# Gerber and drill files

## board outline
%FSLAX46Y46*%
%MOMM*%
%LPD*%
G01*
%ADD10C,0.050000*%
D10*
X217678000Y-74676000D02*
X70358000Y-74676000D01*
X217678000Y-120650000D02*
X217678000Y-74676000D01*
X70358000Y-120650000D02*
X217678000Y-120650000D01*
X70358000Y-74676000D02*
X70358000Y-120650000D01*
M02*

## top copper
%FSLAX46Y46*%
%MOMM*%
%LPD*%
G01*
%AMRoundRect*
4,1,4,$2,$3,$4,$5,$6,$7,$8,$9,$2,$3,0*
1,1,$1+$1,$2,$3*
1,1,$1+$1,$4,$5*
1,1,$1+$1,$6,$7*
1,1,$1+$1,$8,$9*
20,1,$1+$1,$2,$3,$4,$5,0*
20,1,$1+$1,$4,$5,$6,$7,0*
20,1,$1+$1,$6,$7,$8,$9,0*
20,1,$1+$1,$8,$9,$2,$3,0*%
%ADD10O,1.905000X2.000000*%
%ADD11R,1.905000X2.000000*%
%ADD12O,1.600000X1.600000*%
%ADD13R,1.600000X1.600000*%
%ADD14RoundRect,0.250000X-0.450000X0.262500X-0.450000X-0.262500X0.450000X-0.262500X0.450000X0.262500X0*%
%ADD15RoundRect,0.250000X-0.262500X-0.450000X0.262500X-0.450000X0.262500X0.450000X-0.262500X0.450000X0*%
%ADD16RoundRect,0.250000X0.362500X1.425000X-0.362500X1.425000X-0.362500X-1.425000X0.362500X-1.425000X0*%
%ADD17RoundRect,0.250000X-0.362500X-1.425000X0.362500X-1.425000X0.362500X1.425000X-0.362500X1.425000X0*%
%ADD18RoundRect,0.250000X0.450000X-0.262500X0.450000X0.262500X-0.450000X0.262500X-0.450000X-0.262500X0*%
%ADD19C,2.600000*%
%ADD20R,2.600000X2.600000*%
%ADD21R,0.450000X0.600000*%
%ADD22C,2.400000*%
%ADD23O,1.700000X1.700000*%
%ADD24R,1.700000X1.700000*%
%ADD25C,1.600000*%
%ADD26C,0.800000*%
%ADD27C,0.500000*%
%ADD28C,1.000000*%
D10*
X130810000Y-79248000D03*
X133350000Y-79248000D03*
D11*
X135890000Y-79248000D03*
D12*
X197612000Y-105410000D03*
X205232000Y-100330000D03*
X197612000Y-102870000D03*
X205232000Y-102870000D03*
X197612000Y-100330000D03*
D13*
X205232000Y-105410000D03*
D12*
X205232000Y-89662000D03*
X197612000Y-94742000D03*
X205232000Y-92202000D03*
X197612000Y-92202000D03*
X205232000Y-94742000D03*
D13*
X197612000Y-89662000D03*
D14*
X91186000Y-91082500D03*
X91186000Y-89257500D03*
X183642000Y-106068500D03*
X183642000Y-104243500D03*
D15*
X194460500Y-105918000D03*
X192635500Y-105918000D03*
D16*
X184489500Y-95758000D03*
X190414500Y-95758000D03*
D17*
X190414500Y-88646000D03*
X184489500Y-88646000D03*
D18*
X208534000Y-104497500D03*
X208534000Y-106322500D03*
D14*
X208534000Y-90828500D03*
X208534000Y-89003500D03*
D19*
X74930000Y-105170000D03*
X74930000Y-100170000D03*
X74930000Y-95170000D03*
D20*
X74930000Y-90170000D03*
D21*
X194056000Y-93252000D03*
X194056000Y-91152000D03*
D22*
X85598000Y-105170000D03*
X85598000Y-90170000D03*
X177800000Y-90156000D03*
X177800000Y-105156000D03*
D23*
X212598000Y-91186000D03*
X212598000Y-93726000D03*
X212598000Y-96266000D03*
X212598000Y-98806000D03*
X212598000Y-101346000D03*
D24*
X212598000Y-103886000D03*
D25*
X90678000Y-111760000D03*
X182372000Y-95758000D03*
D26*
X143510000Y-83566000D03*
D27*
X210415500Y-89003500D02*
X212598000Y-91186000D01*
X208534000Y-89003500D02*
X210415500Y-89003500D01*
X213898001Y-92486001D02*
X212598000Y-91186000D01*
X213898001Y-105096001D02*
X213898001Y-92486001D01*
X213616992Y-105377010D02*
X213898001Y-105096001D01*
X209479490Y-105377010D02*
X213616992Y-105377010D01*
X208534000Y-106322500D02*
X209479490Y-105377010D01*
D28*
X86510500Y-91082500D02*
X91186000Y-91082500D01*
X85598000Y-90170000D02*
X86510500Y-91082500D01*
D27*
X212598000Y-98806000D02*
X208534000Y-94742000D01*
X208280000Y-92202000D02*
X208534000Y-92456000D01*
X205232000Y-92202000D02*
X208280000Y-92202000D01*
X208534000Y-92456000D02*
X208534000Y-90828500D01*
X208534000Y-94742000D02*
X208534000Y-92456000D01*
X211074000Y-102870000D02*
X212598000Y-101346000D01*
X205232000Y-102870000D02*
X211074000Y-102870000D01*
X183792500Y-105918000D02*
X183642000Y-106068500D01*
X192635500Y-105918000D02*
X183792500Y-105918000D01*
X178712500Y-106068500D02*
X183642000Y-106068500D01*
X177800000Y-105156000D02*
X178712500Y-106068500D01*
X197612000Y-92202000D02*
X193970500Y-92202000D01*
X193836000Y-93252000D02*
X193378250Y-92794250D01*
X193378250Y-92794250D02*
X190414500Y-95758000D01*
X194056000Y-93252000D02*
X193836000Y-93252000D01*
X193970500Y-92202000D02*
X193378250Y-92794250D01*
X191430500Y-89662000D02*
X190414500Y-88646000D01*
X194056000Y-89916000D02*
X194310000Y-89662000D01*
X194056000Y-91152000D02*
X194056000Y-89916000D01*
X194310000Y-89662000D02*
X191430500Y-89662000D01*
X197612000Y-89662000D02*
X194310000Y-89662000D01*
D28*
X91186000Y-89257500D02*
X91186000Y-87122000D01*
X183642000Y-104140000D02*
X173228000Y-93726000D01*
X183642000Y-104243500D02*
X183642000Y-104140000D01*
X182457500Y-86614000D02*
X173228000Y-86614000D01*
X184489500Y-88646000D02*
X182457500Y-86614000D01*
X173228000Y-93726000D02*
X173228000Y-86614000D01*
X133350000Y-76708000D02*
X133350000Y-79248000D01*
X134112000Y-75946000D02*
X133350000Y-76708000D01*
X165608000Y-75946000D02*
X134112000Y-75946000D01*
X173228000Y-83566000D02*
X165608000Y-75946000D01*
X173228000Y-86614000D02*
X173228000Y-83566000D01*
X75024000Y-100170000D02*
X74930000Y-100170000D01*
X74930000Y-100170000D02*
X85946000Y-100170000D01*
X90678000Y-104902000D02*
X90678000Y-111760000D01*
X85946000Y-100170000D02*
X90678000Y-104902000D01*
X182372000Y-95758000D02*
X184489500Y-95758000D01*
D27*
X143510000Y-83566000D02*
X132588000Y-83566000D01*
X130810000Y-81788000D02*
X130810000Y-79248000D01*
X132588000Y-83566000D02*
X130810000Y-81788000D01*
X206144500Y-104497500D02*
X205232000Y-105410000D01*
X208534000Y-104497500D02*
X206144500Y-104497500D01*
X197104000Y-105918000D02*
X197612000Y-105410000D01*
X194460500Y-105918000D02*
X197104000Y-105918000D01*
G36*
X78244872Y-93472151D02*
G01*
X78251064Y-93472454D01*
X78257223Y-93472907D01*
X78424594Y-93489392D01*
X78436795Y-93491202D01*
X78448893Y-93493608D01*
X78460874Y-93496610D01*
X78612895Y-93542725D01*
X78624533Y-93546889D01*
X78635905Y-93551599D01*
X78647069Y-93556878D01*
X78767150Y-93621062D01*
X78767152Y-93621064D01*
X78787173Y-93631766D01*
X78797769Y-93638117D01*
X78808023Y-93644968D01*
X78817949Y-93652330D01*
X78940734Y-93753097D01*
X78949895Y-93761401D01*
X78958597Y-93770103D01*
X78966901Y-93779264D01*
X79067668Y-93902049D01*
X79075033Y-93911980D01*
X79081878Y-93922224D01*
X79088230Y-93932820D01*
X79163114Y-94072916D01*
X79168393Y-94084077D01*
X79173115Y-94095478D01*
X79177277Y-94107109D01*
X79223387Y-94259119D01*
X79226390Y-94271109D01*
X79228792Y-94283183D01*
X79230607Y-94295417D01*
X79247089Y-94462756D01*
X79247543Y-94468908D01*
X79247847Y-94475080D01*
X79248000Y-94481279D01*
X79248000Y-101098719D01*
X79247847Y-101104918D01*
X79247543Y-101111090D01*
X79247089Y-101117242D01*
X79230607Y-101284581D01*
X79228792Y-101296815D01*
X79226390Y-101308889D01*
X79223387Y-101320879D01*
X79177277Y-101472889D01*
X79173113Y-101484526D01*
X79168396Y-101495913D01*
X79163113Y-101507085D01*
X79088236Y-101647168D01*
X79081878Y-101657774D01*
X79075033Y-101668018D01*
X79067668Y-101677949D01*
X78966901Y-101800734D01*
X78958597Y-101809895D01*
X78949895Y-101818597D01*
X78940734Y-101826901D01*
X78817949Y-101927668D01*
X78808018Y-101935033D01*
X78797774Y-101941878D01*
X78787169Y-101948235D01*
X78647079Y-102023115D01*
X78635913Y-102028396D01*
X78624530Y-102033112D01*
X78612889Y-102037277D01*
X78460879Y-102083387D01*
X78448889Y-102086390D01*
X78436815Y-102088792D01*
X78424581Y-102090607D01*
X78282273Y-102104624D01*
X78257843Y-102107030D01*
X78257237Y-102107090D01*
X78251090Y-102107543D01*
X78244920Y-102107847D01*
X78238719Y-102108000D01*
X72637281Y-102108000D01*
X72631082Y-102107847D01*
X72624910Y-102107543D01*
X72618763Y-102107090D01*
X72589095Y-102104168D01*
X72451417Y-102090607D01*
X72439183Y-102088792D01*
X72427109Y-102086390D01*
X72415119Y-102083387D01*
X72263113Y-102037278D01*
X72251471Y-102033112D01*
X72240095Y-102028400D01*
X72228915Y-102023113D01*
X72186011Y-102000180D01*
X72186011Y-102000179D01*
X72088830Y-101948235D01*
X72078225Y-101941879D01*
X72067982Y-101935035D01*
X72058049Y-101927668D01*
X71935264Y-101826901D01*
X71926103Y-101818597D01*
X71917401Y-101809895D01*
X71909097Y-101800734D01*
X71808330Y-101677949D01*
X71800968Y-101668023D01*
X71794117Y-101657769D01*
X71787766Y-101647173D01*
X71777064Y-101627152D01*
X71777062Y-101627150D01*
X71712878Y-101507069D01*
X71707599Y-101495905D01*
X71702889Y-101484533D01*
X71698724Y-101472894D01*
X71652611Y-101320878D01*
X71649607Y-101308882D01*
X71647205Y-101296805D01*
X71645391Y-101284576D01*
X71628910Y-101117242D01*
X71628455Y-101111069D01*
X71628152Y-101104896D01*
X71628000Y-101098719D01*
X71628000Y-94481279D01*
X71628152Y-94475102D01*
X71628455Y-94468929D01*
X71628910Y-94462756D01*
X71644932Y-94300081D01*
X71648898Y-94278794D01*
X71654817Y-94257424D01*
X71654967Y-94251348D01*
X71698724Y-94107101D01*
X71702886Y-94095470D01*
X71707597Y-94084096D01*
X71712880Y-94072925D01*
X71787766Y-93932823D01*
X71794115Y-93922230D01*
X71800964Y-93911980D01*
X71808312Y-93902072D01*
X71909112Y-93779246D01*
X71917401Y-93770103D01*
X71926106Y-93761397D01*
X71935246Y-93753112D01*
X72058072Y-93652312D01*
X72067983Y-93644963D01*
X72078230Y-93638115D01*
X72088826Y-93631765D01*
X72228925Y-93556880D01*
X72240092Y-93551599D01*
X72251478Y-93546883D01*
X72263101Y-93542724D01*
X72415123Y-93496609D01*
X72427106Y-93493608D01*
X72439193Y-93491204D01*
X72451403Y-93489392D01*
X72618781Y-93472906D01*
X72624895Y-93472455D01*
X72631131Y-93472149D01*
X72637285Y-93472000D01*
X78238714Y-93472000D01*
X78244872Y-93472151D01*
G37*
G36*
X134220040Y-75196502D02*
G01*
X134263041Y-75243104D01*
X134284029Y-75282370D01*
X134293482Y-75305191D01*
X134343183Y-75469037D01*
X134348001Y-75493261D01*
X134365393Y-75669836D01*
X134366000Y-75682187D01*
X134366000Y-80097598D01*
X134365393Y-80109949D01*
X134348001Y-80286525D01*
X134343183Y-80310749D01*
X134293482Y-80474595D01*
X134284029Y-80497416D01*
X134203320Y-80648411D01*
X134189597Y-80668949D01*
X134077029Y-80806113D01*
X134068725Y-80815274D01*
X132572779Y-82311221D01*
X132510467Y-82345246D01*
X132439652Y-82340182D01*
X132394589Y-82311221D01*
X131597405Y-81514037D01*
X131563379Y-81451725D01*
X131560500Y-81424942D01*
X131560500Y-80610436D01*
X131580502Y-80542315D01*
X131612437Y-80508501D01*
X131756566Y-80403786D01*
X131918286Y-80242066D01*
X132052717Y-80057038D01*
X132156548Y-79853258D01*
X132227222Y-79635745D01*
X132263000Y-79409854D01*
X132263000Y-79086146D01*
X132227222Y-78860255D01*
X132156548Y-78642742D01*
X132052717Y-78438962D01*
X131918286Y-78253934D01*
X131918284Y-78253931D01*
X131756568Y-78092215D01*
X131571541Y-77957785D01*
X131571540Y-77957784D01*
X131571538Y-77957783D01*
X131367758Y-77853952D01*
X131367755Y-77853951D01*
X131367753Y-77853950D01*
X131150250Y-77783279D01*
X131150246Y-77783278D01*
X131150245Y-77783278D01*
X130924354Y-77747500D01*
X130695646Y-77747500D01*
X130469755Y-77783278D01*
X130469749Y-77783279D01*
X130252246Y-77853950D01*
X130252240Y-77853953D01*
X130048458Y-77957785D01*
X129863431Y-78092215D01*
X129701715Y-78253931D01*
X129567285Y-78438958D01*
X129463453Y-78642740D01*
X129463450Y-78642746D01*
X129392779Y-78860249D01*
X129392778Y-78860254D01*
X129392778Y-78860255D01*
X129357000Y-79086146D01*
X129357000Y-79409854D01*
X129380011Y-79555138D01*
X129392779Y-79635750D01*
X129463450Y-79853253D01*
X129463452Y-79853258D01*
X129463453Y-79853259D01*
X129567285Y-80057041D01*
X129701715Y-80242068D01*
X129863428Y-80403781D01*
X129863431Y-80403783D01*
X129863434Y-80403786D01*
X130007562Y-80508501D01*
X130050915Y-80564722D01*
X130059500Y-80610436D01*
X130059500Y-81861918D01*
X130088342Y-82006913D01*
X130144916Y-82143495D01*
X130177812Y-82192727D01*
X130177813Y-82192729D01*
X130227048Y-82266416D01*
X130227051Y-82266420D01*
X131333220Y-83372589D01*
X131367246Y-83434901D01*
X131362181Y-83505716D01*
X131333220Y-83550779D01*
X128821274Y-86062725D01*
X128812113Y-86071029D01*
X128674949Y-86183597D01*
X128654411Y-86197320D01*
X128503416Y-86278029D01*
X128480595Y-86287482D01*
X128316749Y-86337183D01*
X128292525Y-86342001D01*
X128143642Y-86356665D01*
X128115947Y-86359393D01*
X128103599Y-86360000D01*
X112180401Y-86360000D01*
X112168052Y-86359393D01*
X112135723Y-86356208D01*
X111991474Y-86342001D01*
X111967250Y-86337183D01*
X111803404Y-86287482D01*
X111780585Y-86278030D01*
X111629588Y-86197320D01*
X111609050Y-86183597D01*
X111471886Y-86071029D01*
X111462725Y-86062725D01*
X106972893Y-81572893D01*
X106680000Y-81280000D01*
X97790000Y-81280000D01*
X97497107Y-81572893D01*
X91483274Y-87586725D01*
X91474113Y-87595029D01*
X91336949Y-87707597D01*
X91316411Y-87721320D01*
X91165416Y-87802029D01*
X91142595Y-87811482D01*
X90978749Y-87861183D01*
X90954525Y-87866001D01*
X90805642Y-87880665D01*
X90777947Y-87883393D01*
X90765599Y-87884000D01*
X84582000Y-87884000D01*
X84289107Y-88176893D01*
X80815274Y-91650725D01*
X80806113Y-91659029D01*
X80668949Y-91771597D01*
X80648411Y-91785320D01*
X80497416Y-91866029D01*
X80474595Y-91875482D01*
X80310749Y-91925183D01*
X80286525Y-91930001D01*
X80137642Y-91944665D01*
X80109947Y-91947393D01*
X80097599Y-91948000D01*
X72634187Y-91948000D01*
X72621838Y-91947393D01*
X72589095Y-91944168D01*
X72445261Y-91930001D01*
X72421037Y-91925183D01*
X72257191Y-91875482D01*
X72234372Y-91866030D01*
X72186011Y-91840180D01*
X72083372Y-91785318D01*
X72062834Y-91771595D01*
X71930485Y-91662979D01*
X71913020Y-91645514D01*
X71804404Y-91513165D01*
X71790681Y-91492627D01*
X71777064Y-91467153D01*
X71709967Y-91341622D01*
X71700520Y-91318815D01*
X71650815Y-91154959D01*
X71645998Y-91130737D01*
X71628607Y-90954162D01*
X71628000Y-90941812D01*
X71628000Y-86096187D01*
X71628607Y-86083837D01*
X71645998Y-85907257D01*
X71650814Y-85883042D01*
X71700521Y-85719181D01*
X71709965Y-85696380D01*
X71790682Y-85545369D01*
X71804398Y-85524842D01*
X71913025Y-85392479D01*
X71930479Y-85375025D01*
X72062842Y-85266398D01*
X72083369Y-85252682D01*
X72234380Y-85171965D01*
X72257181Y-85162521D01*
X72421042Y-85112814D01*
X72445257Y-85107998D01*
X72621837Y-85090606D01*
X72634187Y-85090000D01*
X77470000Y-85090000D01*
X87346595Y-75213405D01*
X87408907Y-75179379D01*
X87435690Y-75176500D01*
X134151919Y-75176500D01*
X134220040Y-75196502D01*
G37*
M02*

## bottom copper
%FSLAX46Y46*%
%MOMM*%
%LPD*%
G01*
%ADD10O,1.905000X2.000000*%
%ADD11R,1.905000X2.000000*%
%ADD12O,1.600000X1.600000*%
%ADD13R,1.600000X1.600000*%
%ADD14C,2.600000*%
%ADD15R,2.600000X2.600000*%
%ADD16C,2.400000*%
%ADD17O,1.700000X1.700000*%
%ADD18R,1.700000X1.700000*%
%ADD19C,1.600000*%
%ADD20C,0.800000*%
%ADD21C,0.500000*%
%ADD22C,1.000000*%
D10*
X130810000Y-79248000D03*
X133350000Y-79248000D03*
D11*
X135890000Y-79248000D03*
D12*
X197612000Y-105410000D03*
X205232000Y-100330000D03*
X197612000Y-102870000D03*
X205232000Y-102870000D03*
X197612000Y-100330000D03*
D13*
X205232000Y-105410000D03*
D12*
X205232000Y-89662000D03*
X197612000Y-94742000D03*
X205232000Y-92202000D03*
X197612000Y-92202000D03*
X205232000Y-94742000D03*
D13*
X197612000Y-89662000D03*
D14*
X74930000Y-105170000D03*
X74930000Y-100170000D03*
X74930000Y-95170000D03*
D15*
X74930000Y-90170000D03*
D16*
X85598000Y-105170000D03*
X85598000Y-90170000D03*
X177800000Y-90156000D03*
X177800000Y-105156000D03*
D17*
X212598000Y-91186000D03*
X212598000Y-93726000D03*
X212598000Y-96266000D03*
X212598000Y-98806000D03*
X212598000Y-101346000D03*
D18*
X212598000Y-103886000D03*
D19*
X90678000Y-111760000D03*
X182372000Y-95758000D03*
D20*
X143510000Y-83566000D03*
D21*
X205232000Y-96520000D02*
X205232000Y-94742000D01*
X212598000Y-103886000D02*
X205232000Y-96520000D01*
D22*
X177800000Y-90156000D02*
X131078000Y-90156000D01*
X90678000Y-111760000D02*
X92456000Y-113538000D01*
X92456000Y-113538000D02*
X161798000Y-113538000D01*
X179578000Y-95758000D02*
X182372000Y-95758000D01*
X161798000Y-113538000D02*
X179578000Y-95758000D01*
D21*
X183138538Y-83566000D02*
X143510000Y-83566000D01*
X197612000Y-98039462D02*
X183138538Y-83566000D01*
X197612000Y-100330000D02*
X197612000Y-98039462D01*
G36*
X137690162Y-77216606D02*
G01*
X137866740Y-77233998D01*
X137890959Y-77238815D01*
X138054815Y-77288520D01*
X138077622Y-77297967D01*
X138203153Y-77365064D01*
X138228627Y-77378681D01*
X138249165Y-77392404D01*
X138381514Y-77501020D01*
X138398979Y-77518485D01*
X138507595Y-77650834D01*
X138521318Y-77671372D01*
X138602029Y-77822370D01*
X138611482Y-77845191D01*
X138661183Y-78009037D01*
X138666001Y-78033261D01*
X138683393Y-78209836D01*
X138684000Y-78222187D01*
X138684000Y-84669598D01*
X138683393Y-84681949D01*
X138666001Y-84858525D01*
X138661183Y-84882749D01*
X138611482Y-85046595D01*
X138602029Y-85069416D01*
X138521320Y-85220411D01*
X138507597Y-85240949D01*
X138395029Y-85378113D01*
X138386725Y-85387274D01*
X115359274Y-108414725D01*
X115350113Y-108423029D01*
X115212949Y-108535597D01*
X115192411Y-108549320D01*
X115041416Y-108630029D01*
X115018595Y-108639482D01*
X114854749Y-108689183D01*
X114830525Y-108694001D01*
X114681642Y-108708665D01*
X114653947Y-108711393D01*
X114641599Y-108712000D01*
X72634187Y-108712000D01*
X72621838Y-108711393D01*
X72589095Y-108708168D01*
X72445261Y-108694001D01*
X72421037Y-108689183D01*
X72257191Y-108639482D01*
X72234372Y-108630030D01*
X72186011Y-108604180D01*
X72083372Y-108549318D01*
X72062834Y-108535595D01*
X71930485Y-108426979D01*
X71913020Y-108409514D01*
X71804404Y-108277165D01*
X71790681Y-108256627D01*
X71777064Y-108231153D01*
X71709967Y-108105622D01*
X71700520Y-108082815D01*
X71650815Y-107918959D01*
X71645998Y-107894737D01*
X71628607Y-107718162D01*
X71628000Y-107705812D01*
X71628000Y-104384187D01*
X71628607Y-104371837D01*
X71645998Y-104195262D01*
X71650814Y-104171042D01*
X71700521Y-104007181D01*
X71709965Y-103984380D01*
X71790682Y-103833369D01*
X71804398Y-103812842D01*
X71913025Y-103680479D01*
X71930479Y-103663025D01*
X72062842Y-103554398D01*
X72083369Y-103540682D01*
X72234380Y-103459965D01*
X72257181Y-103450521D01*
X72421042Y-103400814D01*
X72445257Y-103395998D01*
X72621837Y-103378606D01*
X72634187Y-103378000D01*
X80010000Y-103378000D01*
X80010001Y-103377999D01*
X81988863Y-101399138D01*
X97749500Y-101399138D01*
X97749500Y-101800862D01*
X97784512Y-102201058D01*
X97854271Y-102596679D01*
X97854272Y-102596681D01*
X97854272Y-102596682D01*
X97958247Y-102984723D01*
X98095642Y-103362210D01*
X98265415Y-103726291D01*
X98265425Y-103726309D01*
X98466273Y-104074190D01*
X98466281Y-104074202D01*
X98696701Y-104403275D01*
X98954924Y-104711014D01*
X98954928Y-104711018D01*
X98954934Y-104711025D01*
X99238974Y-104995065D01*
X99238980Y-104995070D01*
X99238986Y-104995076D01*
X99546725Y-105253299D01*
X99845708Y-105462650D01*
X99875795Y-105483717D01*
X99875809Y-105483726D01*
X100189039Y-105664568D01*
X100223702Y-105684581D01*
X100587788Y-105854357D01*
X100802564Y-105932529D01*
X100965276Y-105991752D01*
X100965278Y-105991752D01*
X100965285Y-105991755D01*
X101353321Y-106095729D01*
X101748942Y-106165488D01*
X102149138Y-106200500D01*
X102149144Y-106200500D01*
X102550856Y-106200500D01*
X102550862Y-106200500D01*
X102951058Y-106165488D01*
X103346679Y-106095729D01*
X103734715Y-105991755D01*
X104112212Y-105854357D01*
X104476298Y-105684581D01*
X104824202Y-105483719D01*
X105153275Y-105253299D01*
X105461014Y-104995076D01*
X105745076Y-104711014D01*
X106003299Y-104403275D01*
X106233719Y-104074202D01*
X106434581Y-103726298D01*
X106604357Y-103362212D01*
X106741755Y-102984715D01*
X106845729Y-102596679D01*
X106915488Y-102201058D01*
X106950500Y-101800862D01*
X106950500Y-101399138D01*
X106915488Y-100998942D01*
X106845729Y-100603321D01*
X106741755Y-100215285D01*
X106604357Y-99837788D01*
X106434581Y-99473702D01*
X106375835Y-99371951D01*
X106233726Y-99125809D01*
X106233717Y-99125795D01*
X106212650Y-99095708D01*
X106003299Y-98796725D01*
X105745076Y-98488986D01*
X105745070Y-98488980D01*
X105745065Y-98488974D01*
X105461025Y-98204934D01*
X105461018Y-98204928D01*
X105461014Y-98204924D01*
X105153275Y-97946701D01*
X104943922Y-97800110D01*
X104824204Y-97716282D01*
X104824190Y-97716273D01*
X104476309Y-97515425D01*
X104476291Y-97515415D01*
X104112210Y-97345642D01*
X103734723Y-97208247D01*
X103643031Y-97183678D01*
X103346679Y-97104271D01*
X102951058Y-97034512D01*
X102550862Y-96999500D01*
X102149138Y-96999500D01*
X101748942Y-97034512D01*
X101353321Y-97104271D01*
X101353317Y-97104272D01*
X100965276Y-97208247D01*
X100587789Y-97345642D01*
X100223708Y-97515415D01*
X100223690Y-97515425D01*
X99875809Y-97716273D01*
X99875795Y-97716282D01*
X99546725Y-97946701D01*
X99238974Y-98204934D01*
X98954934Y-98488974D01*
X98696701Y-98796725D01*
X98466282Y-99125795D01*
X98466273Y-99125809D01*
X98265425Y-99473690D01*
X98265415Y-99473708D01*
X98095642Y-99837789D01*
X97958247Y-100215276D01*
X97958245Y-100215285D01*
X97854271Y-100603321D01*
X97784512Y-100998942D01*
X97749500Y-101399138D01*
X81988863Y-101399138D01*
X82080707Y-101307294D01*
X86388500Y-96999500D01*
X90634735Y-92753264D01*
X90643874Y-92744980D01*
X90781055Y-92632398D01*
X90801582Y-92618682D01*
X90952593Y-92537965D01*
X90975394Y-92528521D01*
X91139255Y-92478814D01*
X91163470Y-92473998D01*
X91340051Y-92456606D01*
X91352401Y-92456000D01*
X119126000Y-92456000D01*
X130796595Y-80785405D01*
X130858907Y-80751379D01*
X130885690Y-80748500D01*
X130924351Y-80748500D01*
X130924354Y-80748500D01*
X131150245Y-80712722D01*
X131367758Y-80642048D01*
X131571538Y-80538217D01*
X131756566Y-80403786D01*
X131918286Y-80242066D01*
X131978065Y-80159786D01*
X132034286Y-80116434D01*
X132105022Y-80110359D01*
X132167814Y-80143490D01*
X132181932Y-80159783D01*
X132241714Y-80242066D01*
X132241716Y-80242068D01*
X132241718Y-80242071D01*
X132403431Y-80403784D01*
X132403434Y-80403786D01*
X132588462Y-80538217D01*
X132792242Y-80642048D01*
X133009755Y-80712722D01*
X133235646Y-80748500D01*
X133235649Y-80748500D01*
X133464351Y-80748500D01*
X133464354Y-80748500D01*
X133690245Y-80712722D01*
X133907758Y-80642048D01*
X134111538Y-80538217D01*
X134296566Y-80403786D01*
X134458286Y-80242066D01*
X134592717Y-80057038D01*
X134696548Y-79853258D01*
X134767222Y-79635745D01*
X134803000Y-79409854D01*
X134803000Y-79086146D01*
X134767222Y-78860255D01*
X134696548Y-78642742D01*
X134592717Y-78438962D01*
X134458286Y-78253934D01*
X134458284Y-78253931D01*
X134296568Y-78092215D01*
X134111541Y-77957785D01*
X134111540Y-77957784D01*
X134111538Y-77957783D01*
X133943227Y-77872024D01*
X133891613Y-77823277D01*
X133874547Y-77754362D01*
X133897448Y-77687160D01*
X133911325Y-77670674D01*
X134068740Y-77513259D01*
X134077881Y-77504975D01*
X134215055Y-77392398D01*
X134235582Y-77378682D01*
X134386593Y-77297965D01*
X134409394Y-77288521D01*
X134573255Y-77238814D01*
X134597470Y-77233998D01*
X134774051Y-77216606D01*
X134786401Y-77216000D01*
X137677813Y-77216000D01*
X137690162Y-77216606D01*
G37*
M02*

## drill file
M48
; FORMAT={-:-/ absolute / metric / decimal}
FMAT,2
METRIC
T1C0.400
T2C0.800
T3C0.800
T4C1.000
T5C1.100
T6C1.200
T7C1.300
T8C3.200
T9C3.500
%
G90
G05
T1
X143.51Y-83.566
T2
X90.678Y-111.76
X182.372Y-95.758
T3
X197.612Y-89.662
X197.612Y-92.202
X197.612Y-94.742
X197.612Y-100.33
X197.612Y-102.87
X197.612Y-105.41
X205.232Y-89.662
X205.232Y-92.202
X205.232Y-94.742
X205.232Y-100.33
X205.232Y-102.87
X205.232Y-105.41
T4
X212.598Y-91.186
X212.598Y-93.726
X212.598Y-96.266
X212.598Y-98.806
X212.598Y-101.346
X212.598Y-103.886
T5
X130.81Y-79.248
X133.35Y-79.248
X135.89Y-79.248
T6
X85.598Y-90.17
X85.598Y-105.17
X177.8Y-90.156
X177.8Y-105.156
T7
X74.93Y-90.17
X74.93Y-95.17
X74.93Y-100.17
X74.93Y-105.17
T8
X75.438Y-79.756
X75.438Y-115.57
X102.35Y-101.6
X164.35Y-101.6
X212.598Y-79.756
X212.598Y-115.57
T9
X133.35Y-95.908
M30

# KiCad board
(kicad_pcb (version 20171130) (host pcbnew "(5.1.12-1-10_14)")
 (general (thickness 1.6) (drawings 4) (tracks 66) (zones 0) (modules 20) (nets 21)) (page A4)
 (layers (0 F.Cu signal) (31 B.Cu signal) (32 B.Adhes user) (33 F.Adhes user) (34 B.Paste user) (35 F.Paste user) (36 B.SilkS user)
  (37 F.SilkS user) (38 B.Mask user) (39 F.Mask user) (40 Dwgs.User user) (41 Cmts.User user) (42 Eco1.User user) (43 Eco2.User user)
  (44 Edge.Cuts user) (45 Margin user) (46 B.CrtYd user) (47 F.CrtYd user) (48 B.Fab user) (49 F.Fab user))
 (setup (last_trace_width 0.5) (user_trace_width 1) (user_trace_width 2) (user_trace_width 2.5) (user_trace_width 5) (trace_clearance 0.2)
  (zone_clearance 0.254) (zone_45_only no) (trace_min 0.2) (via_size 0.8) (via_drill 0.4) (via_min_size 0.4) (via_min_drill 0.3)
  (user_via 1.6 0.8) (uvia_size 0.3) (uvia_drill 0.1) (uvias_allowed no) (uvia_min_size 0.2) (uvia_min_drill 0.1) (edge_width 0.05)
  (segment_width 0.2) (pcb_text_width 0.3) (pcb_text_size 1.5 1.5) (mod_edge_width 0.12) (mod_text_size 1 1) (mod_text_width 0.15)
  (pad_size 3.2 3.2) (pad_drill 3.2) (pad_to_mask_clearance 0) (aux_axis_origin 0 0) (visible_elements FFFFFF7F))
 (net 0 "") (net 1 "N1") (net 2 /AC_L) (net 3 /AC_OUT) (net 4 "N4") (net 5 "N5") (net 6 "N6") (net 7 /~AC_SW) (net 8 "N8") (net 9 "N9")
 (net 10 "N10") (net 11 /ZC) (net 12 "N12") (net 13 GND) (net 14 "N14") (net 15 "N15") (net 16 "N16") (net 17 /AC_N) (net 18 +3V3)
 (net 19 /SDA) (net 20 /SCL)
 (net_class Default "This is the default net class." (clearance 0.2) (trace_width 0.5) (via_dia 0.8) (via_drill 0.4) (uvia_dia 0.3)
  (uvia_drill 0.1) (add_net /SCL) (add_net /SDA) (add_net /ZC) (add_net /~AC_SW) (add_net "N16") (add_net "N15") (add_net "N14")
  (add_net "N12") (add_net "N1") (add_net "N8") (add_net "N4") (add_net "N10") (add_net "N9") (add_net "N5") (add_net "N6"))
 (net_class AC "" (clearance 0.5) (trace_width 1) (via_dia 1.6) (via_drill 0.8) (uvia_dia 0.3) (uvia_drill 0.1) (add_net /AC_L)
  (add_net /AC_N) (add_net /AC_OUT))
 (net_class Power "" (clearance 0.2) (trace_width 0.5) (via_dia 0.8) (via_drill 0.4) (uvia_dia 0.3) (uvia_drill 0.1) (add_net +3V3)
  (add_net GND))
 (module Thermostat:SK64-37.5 (layer F.Cu) (at 133.35 101.6 180)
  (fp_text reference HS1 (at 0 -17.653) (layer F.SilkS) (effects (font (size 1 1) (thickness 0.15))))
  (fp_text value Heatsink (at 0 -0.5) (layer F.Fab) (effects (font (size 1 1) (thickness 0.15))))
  (pad "" np_thru_hole circle (at 31 0 180) (size 3.2 3.2) (drill 3.2) (layers *.Cu *.Mask) (solder_mask_margin 2.4) (clearance 3))
  (pad "" np_thru_hole circle (at -31 0 180) (size 3.2 3.2) (drill 3.2) (layers *.Cu *.Mask) (solder_mask_margin 2.4) (clearance 3)))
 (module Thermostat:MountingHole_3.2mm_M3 (layer F.Cu) (at 212.598 115.57)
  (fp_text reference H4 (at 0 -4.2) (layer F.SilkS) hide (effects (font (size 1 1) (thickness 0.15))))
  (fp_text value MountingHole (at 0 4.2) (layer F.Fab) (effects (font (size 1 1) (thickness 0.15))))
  (pad "" np_thru_hole circle (at 0 0) (size 3.2 3.2) (drill 3.2) (layers *.Cu *.Mask) (solder_mask_margin 2.4) (clearance 3)))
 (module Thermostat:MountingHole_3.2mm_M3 (layer F.Cu) (at 212.598 79.756)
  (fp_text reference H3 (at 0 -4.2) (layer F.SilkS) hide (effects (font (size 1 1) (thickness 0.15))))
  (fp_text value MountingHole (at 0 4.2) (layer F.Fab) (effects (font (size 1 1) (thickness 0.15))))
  (pad "" np_thru_hole circle (at 0 0) (size 3.2 3.2) (drill 3.2) (layers *.Cu *.Mask) (solder_mask_margin 2.4) (clearance 3)))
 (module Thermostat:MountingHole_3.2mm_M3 (layer F.Cu) (at 75.438 115.57)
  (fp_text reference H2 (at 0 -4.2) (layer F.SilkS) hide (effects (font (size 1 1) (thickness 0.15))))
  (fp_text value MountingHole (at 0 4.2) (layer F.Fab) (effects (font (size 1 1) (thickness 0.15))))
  (pad "" np_thru_hole circle (at 0 0) (size 3.2 3.2) (drill 3.2) (layers *.Cu *.Mask) (solder_mask_margin 2.4) (clearance 3)))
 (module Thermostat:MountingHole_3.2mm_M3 (layer F.Cu) (at 75.438 79.756)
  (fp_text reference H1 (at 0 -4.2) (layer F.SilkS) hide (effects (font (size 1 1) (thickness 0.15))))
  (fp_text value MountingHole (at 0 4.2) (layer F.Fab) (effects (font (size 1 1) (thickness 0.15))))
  (pad "" np_thru_hole circle (at 0 0) (size 3.2 3.2) (drill 3.2) (layers *.Cu *.Mask) (solder_mask_margin 2.4) (clearance 3)))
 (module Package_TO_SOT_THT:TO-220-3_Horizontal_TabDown (layer F.Cu) (at 135.89 79.248 180)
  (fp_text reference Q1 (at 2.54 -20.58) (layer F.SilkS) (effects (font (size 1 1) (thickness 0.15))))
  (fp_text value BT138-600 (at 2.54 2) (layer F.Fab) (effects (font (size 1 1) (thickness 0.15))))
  (pad 3 thru_hole oval (at 5.08 0 180) (size 1.905 2) (drill 1.1) (layers *.Cu *.Mask) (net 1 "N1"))
  (pad 2 thru_hole oval (at 2.54 0 180) (size 1.905 2) (drill 1.1) (layers *.Cu *.Mask) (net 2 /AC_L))
  (pad 1 thru_hole rect (at 0 0 180) (size 1.905 2) (drill 1.1) (layers *.Cu *.Mask) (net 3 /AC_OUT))
  (pad "" np_thru_hole oval (at 2.54 -16.66 180) (size 3.5 3.5) (drill 3.5) (layers *.Cu *.Mask)))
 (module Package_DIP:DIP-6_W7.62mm (layer F.Cu) (at 205.232 105.41 180)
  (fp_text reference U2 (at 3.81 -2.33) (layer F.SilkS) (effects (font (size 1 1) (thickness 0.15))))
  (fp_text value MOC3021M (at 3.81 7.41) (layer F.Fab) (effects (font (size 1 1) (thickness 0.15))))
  (pad 6 thru_hole oval (at 7.62 0 180) (size 1.6 1.6) (drill 0.8) (layers *.Cu *.Mask) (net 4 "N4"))
  (pad 3 thru_hole oval (at 0 5.08 180) (size 1.6 1.6) (drill 0.8) (layers *.Cu *.Mask) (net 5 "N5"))
  (pad 5 thru_hole oval (at 7.62 2.54 180) (size 1.6 1.6) (drill 0.8) (layers *.Cu *.Mask) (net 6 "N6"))
  (pad 2 thru_hole oval (at 0 2.54 180) (size 1.6 1.6) (drill 0.8) (layers *.Cu *.Mask) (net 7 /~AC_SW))
  (pad 4 thru_hole oval (at 7.62 5.08 180) (size 1.6 1.6) (drill 0.8) (layers *.Cu *.Mask) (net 1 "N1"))
  (pad 1 thru_hole rect (at 0 0 180) (size 1.6 1.6) (drill 0.8) (layers *.Cu *.Mask) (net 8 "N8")))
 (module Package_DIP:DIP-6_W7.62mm (layer F.Cu) (at 197.612 89.662)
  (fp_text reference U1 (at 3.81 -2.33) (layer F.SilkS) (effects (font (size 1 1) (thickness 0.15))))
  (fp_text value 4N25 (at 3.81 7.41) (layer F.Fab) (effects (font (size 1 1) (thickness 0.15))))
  (pad 6 thru_hole oval (at 7.62 0) (size 1.6 1.6) (drill 0.8) (layers *.Cu *.Mask) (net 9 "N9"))
  (pad 3 thru_hole oval (at 0 5.08) (size 1.6 1.6) (drill 0.8) (layers *.Cu *.Mask) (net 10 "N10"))
  (pad 5 thru_hole oval (at 7.62 2.54) (size 1.6 1.6) (drill 0.8) (layers *.Cu *.Mask) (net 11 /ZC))
  (pad 2 thru_hole oval (at 0 2.54) (size 1.6 1.6) (drill 0.8) (layers *.Cu *.Mask) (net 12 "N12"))
  (pad 4 thru_hole oval (at 7.62 5.08) (size 1.6 1.6) (drill 0.8) (layers *.Cu *.Mask) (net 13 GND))
  (pad 1 thru_hole rect (at 0 0) (size 1.6 1.6) (drill 0.8) (layers *.Cu *.Mask) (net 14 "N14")))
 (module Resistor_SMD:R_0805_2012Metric (layer F.Cu) (at 91.186 90.17 270)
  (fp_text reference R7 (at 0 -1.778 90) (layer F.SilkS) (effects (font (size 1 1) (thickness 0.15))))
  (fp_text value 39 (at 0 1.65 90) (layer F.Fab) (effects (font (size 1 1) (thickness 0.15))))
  (pad 2 smd roundrect (at 0.9125 0 270) (size 1.025 1.4) (layers F.Cu F.Paste F.Mask) (roundrect_rratio 0.243902) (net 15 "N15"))
  (pad 1 smd roundrect (at -0.9125 0 270) (size 1.025 1.4) (layers F.Cu F.Paste F.Mask) (roundrect_rratio 0.243902) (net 2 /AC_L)))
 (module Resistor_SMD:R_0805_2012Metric (layer F.Cu) (at 183.642 105.156 270)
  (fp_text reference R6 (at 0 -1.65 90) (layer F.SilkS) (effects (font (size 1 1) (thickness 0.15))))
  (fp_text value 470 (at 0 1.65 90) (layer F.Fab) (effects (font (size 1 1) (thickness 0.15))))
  (pad 2 smd roundrect (at 0.9125 0 270) (size 1.025 1.4) (layers F.Cu F.Paste F.Mask) (roundrect_rratio 0.243902) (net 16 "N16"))
  (pad 1 smd roundrect (at -0.9125 0 270) (size 1.025 1.4) (layers F.Cu F.Paste F.Mask) (roundrect_rratio 0.243902) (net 2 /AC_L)))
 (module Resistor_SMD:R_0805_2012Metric (layer F.Cu) (at 193.548 105.918)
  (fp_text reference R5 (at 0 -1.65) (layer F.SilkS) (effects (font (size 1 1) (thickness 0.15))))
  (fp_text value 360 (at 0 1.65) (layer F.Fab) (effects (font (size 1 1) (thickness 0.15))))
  (pad 2 smd roundrect (at 0.9125 0) (size 1.025 1.4) (layers F.Cu F.Paste F.Mask) (roundrect_rratio 0.243902) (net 4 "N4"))
  (pad 1 smd roundrect (at -0.9125 0) (size 1.025 1.4) (layers F.Cu F.Paste F.Mask) (roundrect_rratio 0.243902) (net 16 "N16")))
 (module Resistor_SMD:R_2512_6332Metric (layer F.Cu) (at 187.452 95.758 180)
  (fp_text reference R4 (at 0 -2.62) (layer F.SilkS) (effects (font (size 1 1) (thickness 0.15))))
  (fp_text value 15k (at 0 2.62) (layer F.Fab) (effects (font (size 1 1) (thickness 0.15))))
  (pad 2 smd roundrect (at 2.9625 0 180) (size 1.225 3.35) (layers F.Cu F.Paste F.Mask) (roundrect_rratio 0.204082) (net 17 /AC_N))
  (pad 1 smd roundrect (at -2.9625 0 180) (size 1.225 3.35) (layers F.Cu F.Paste F.Mask) (roundrect_rratio 0.204082) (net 12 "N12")))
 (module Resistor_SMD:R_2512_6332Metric (layer F.Cu) (at 187.452 88.646)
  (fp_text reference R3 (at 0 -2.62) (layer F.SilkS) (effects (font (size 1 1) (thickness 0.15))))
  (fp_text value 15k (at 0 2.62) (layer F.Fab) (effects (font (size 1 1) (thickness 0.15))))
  (pad 2 smd roundrect (at 2.9625 0) (size 1.225 3.35) (layers F.Cu F.Paste F.Mask) (roundrect_rratio 0.204082) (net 14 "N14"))
  (pad 1 smd roundrect (at -2.9625 0) (size 1.225 3.35) (layers F.Cu F.Paste F.Mask) (roundrect_rratio 0.204082) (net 2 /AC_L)))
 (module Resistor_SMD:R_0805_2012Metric (layer F.Cu) (at 208.534 105.41 90)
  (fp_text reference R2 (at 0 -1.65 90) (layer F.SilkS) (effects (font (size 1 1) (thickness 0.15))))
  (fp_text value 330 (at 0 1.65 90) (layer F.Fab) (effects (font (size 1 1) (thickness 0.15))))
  (pad 2 smd roundrect (at 0.9125 0 90) (size 1.025 1.4) (layers F.Cu F.Paste F.Mask) (roundrect_rratio 0.243902) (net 8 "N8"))
  (pad 1 smd roundrect (at -0.9125 0 90) (size 1.025 1.4) (layers F.Cu F.Paste F.Mask) (roundrect_rratio 0.243902) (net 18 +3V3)))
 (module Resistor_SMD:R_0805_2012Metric (layer F.Cu) (at 208.534 89.916 270)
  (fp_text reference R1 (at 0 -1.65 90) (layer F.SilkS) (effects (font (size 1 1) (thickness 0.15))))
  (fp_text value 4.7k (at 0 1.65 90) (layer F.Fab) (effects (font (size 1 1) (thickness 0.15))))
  (pad 2 smd roundrect (at 0.9125 0 270) (size 1.025 1.4) (layers F.Cu F.Paste F.Mask) (roundrect_rratio 0.243902) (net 11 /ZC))
  (pad 1 smd roundrect (at -0.9125 0 270) (size 1.025 1.4) (layers F.Cu F.Paste F.Mask) (roundrect_rratio 0.243902) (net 18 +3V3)))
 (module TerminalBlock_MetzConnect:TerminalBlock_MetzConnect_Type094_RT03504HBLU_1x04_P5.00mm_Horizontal (layer F.Cu) (at 74.93 90.17 270)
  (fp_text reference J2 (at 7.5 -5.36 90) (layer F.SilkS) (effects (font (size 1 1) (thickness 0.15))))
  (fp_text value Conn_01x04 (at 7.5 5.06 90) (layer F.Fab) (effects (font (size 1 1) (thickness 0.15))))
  (pad 4 thru_hole circle (at 15 0 270) (size 2.6 2.6) (drill 1.3) (layers *.Cu *.Mask) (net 3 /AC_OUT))
  (pad 3 thru_hole circle (at 10 0 270) (size 2.6 2.6) (drill 1.3) (layers *.Cu *.Mask) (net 17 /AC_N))
  (pad 2 thru_hole circle (at 5 0 270) (size 2.6 2.6) (drill 1.3) (layers *.Cu *.Mask) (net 17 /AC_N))
  (pad 1 thru_hole rect (at 0 0 270) (size 2.6 2.6) (drill 1.3) (layers *.Cu *.Mask) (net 2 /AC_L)))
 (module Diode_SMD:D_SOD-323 (layer F.Cu) (at 194.056 92.202 270)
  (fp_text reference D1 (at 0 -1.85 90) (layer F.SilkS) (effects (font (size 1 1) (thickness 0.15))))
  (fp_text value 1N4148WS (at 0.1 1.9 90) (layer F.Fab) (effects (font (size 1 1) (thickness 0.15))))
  (pad 2 smd rect (at 1.05 0 270) (size 0.6 0.45) (layers F.Cu F.Paste F.Mask) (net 12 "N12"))
  (pad 1 smd rect (at -1.05 0 270) (size 0.6 0.45) (layers F.Cu F.Paste F.Mask) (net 14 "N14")))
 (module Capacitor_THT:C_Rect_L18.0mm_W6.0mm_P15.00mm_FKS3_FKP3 (layer F.Cu) (at 85.598 90.17 270)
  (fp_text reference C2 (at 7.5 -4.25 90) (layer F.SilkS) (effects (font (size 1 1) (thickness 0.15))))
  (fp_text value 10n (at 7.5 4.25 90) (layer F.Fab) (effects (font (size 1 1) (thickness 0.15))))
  (pad 2 thru_hole circle (at 15 0 270) (size 2.4 2.4) (drill 1.2) (layers *.Cu *.Mask) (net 3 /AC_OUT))
  (pad 1 thru_hole circle (at 0 0 270) (size 2.4 2.4) (drill 1.2) (layers *.Cu *.Mask) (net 15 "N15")))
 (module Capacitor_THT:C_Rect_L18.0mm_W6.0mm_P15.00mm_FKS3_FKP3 (layer F.Cu) (at 177.8 105.156 90)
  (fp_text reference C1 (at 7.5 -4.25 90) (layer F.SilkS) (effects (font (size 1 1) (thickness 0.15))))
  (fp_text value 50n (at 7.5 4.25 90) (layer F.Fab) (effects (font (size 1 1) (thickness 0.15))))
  (pad 2 thru_hole circle (at 15 0 90) (size 2.4 2.4) (drill 1.2) (layers *.Cu *.Mask) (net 3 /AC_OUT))
  (pad 1 thru_hole circle (at 0 0 90) (size 2.4 2.4) (drill 1.2) (layers *.Cu *.Mask) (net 16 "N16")))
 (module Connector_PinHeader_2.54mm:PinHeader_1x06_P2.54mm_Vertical (layer B.Cu) (at 212.598 103.886)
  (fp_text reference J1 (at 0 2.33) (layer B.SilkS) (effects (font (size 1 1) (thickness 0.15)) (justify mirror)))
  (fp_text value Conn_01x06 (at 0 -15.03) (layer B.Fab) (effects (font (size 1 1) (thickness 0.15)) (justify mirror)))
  (pad 6 thru_hole oval (at 0 -12.7) (size 1.7 1.7) (drill 1) (layers *.Cu *.Mask) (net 18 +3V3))
  (pad 5 thru_hole oval (at 0 -10.16) (size 1.7 1.7) (drill 1) (layers *.Cu *.Mask) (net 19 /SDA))
  (pad 4 thru_hole oval (at 0 -7.62) (size 1.7 1.7) (drill 1) (layers *.Cu *.Mask) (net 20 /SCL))
  (pad 3 thru_hole oval (at 0 -5.08) (size 1.7 1.7) (drill 1) (layers *.Cu *.Mask) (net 11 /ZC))
  (pad 2 thru_hole oval (at 0 -2.54) (size 1.7 1.7) (drill 1) (layers *.Cu *.Mask) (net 7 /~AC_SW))
  (pad 1 thru_hole rect (at 0 0) (size 1.7 1.7) (drill 1) (layers *.Cu *.Mask) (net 13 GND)))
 (gr_line (start 217.678 74.676) (end 70.358 74.676) (layer Edge.Cuts) (width 0.05))
 (gr_line (start 217.678 120.65) (end 217.678 74.676) (layer Edge.Cuts) (width 0.05))
 (gr_line (start 70.358 120.65) (end 217.678 120.65) (layer Edge.Cuts) (width 0.05))
 (gr_line (start 70.358 74.676) (end 70.358 120.65) (layer Edge.Cuts) (width 0.05))
 (segment (start 205.232 96.52) (end 205.232 94.742) (width 0.5) (layer B.Cu) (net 13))
 (segment (start 212.598 103.886) (end 205.232 96.52) (width 0.5) (layer B.Cu) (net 13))
 (segment (start 210.4155 89.0035) (end 212.598 91.186) (width 0.5) (layer F.Cu) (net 18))
 (segment (start 208.534 89.0035) (end 210.4155 89.0035) (width 0.5) (layer F.Cu) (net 18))
 (segment (start 213.898001 92.486001) (end 212.598 91.186) (width 0.5) (layer F.Cu) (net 18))
 (segment (start 213.898001 105.096001) (end 213.898001 92.486001) (width 0.5) (layer F.Cu) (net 18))
 (segment (start 213.616992 105.37701) (end 213.898001 105.096001) (width 0.5) (layer F.Cu) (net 18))
 (segment (start 209.47949 105.37701) (end 213.616992 105.37701) (width 0.5) (layer F.Cu) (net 18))
 (segment (start 208.534 106.3225) (end 209.47949 105.37701) (width 0.5) (layer F.Cu) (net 18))
 (segment (start 86.5105 91.0825) (end 91.186 91.0825) (width 1) (layer F.Cu) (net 15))
 (segment (start 85.598 90.17) (end 86.5105 91.0825) (width 1) (layer F.Cu) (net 15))
 (segment (start 212.598 98.806) (end 208.534 94.742) (width 0.5) (layer F.Cu) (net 11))
 (segment (start 208.28 92.202) (end 208.534 92.456) (width 0.5) (layer F.Cu) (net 11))
 (segment (start 205.232 92.202) (end 208.28 92.202) (width 0.5) (layer F.Cu) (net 11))
 (segment (start 208.534 92.456) (end 208.534 90.8285) (width 0.5) (layer F.Cu) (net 11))
 (segment (start 208.534 94.742) (end 208.534 92.456) (width 0.5) (layer F.Cu) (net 11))
 (segment (start 211.074 102.87) (end 212.598 101.346) (width 0.5) (layer F.Cu) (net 7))
 (segment (start 205.232 102.87) (end 211.074 102.87) (width 0.5) (layer F.Cu) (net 7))
 (segment (start 177.8 90.156) (end 131.078 90.156) (width 1) (layer B.Cu) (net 3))
 (segment (start 183.7925 105.918) (end 183.642 106.0685) (width 0.5) (layer F.Cu) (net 16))
 (segment (start 192.6355 105.918) (end 183.7925 105.918) (width 0.5) (layer F.Cu) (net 16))
 (segment (start 178.7125 106.0685) (end 183.642 106.0685) (width 0.5) (layer F.Cu) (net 16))
 (segment (start 177.8 105.156) (end 178.7125 106.0685) (width 0.5) (layer F.Cu) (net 16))
 (segment (start 197.612 92.202) (end 193.9705 92.202) (width 0.5) (layer F.Cu) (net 12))
 (segment (start 193.836 93.252) (end 193.37825 92.79425) (width 0.5) (layer F.Cu) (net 12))
 (segment (start 193.37825 92.79425) (end 190.4145 95.758) (width 0.5) (layer F.Cu) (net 12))
 (segment (start 194.056 93.252) (end 193.836 93.252) (width 0.5) (layer F.Cu) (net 12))
 (segment (start 193.9705 92.202) (end 193.37825 92.79425) (width 0.5) (layer F.Cu) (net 12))
 (segment (start 191.4305 89.662) (end 190.4145 88.646) (width 0.5) (layer F.Cu) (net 14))
 (segment (start 194.056 89.916) (end 194.31 89.662) (width 0.5) (layer F.Cu) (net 14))
 (segment (start 194.056 91.152) (end 194.056 89.916) (width 0.5) (layer F.Cu) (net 14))
 (segment (start 194.31 89.662) (end 191.4305 89.662) (width 0.5) (layer F.Cu) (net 14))
 (segment (start 197.612 89.662) (end 194.31 89.662) (width 0.5) (layer F.Cu) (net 14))
 (segment (start 91.186 89.2575) (end 91.186 87.122) (width 1) (layer F.Cu) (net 2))
 (segment (start 183.642 104.14) (end 173.228 93.726) (width 1) (layer F.Cu) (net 2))
 (segment (start 183.642 104.2435) (end 183.642 104.14) (width 1) (layer F.Cu) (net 2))
 (segment (start 182.4575 86.614) (end 173.228 86.614) (width 1) (layer F.Cu) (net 2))
 (segment (start 184.4895 88.646) (end 182.4575 86.614) (width 1) (layer F.Cu) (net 2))
 (segment (start 173.228 93.726) (end 173.228 86.614) (width 1) (layer F.Cu) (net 2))
 (segment (start 133.35 76.708) (end 133.35 79.248) (width 1) (layer F.Cu) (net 2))
 (segment (start 134.112 75.946) (end 133.35 76.708) (width 1) (layer F.Cu) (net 2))
 (segment (start 165.608 75.946) (end 134.112 75.946) (width 1) (layer F.Cu) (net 2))
 (segment (start 173.228 83.566) (end 165.608 75.946) (width 1) (layer F.Cu) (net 2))
 (segment (start 173.228 86.614) (end 173.228 83.566) (width 1) (layer F.Cu) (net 2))
 (segment (start 75.024 100.17) (end 74.93 100.17) (width 1) (layer F.Cu) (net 17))
 (segment (start 74.93 100.17) (end 85.946 100.17) (width 1) (layer F.Cu) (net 17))
 (via (at 90.678 111.76) (size 1.6) (drill 0.8) (layers F.Cu B.Cu) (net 17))
 (segment (start 90.678 104.902) (end 90.678 111.76) (width 1) (layer F.Cu) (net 17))
 (segment (start 85.946 100.17) (end 90.678 104.902) (width 1) (layer F.Cu) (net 17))
 (segment (start 90.678 111.76) (end 92.456 113.538) (width 1) (layer B.Cu) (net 17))
 (segment (start 92.456 113.538) (end 161.798 113.538) (width 1) (layer B.Cu) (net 17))
 (via (at 182.372 95.758) (size 1.6) (drill 0.8) (layers F.Cu B.Cu) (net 17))
 (segment (start 179.578 95.758) (end 182.372 95.758) (width 1) (layer B.Cu) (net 17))
 (segment (start 161.798 113.538) (end 179.578 95.758) (width 1) (layer B.Cu) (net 17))
 (segment (start 182.372 95.758) (end 184.4895 95.758) (width 1) (layer F.Cu) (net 17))
 (via (at 143.51 83.566) (size 0.8) (drill 0.4) (layers F.Cu B.Cu) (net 1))
 (segment (start 183.138538 83.566) (end 143.51 83.566) (width 0.5) (layer B.Cu) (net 1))
 (segment (start 197.612 98.039462) (end 183.138538 83.566) (width 0.5) (layer B.Cu) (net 1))
 (segment (start 197.612 100.33) (end 197.612 98.039462) (width 0.5) (layer B.Cu) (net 1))
 (segment (start 143.51 83.566) (end 132.588 83.566) (width 0.5) (layer F.Cu) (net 1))
 (segment (start 130.81 81.788) (end 130.81 79.248) (width 0.5) (layer F.Cu) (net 1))
 (segment (start 132.588 83.566) (end 130.81 81.788) (width 0.5) (layer F.Cu) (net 1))
 (segment (start 206.1445 104.4975) (end 205.232 105.41) (width 0.5) (layer F.Cu) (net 8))
 (segment (start 208.534 104.4975) (end 206.1445 104.4975) (width 0.5) (layer F.Cu) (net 8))
 (segment (start 197.104 105.918) (end 197.612 105.41) (width 0.5) (layer F.Cu) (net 4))
 (segment (start 194.4605 105.918) (end 197.104 105.918) (width 0.5) (layer F.Cu) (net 4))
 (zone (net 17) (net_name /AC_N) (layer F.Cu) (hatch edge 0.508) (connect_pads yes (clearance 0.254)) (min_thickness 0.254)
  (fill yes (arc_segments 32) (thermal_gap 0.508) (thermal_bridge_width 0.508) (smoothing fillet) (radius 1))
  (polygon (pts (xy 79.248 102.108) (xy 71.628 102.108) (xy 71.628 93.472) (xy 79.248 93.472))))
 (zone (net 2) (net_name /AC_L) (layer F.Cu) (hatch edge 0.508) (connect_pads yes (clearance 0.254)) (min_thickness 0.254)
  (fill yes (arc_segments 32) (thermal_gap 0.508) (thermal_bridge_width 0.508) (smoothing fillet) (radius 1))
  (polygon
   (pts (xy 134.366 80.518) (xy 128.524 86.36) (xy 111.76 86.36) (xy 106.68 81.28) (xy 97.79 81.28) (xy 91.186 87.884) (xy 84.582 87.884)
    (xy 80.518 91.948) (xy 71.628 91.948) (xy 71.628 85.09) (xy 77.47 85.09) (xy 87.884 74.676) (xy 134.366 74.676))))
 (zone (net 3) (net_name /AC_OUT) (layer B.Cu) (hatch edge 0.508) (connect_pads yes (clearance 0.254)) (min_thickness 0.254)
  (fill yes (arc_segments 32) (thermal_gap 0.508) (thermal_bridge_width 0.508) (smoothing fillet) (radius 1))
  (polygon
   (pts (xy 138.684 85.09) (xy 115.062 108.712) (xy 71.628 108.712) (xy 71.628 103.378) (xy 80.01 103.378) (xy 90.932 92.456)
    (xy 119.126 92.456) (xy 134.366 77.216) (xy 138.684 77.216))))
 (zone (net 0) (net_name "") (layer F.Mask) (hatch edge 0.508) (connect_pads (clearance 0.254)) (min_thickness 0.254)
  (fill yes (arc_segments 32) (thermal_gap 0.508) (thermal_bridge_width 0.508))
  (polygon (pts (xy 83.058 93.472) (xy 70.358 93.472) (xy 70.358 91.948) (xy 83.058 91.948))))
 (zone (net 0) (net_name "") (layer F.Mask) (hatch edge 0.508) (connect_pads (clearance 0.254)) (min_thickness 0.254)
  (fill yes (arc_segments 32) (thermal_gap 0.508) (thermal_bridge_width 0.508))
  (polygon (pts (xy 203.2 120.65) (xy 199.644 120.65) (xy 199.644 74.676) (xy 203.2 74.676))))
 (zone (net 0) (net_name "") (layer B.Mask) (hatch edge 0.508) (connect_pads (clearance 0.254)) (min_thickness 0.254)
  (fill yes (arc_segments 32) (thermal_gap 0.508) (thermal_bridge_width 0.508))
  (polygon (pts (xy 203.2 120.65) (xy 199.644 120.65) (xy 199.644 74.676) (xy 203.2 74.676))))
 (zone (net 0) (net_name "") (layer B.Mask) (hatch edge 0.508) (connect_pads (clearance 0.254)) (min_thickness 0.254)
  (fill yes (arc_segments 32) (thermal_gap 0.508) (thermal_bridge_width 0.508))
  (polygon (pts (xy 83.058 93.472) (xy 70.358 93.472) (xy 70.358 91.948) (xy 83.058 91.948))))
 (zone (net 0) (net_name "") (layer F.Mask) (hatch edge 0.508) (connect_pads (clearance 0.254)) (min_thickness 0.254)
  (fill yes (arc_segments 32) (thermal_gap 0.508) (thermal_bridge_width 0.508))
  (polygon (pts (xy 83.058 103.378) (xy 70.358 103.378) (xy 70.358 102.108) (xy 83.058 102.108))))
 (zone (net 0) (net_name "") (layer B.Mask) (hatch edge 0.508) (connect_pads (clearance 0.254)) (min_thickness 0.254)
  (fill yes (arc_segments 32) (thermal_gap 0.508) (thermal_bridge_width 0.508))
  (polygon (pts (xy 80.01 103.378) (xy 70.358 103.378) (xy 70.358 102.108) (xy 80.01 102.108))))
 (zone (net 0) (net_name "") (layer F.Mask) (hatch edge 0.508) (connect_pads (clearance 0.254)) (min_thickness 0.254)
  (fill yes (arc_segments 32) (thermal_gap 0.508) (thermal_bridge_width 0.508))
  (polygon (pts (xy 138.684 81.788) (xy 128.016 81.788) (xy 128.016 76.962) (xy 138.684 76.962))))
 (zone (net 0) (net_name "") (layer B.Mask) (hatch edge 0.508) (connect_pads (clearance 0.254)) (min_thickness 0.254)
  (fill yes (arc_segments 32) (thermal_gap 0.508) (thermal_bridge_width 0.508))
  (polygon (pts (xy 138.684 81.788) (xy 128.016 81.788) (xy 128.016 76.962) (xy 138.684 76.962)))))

